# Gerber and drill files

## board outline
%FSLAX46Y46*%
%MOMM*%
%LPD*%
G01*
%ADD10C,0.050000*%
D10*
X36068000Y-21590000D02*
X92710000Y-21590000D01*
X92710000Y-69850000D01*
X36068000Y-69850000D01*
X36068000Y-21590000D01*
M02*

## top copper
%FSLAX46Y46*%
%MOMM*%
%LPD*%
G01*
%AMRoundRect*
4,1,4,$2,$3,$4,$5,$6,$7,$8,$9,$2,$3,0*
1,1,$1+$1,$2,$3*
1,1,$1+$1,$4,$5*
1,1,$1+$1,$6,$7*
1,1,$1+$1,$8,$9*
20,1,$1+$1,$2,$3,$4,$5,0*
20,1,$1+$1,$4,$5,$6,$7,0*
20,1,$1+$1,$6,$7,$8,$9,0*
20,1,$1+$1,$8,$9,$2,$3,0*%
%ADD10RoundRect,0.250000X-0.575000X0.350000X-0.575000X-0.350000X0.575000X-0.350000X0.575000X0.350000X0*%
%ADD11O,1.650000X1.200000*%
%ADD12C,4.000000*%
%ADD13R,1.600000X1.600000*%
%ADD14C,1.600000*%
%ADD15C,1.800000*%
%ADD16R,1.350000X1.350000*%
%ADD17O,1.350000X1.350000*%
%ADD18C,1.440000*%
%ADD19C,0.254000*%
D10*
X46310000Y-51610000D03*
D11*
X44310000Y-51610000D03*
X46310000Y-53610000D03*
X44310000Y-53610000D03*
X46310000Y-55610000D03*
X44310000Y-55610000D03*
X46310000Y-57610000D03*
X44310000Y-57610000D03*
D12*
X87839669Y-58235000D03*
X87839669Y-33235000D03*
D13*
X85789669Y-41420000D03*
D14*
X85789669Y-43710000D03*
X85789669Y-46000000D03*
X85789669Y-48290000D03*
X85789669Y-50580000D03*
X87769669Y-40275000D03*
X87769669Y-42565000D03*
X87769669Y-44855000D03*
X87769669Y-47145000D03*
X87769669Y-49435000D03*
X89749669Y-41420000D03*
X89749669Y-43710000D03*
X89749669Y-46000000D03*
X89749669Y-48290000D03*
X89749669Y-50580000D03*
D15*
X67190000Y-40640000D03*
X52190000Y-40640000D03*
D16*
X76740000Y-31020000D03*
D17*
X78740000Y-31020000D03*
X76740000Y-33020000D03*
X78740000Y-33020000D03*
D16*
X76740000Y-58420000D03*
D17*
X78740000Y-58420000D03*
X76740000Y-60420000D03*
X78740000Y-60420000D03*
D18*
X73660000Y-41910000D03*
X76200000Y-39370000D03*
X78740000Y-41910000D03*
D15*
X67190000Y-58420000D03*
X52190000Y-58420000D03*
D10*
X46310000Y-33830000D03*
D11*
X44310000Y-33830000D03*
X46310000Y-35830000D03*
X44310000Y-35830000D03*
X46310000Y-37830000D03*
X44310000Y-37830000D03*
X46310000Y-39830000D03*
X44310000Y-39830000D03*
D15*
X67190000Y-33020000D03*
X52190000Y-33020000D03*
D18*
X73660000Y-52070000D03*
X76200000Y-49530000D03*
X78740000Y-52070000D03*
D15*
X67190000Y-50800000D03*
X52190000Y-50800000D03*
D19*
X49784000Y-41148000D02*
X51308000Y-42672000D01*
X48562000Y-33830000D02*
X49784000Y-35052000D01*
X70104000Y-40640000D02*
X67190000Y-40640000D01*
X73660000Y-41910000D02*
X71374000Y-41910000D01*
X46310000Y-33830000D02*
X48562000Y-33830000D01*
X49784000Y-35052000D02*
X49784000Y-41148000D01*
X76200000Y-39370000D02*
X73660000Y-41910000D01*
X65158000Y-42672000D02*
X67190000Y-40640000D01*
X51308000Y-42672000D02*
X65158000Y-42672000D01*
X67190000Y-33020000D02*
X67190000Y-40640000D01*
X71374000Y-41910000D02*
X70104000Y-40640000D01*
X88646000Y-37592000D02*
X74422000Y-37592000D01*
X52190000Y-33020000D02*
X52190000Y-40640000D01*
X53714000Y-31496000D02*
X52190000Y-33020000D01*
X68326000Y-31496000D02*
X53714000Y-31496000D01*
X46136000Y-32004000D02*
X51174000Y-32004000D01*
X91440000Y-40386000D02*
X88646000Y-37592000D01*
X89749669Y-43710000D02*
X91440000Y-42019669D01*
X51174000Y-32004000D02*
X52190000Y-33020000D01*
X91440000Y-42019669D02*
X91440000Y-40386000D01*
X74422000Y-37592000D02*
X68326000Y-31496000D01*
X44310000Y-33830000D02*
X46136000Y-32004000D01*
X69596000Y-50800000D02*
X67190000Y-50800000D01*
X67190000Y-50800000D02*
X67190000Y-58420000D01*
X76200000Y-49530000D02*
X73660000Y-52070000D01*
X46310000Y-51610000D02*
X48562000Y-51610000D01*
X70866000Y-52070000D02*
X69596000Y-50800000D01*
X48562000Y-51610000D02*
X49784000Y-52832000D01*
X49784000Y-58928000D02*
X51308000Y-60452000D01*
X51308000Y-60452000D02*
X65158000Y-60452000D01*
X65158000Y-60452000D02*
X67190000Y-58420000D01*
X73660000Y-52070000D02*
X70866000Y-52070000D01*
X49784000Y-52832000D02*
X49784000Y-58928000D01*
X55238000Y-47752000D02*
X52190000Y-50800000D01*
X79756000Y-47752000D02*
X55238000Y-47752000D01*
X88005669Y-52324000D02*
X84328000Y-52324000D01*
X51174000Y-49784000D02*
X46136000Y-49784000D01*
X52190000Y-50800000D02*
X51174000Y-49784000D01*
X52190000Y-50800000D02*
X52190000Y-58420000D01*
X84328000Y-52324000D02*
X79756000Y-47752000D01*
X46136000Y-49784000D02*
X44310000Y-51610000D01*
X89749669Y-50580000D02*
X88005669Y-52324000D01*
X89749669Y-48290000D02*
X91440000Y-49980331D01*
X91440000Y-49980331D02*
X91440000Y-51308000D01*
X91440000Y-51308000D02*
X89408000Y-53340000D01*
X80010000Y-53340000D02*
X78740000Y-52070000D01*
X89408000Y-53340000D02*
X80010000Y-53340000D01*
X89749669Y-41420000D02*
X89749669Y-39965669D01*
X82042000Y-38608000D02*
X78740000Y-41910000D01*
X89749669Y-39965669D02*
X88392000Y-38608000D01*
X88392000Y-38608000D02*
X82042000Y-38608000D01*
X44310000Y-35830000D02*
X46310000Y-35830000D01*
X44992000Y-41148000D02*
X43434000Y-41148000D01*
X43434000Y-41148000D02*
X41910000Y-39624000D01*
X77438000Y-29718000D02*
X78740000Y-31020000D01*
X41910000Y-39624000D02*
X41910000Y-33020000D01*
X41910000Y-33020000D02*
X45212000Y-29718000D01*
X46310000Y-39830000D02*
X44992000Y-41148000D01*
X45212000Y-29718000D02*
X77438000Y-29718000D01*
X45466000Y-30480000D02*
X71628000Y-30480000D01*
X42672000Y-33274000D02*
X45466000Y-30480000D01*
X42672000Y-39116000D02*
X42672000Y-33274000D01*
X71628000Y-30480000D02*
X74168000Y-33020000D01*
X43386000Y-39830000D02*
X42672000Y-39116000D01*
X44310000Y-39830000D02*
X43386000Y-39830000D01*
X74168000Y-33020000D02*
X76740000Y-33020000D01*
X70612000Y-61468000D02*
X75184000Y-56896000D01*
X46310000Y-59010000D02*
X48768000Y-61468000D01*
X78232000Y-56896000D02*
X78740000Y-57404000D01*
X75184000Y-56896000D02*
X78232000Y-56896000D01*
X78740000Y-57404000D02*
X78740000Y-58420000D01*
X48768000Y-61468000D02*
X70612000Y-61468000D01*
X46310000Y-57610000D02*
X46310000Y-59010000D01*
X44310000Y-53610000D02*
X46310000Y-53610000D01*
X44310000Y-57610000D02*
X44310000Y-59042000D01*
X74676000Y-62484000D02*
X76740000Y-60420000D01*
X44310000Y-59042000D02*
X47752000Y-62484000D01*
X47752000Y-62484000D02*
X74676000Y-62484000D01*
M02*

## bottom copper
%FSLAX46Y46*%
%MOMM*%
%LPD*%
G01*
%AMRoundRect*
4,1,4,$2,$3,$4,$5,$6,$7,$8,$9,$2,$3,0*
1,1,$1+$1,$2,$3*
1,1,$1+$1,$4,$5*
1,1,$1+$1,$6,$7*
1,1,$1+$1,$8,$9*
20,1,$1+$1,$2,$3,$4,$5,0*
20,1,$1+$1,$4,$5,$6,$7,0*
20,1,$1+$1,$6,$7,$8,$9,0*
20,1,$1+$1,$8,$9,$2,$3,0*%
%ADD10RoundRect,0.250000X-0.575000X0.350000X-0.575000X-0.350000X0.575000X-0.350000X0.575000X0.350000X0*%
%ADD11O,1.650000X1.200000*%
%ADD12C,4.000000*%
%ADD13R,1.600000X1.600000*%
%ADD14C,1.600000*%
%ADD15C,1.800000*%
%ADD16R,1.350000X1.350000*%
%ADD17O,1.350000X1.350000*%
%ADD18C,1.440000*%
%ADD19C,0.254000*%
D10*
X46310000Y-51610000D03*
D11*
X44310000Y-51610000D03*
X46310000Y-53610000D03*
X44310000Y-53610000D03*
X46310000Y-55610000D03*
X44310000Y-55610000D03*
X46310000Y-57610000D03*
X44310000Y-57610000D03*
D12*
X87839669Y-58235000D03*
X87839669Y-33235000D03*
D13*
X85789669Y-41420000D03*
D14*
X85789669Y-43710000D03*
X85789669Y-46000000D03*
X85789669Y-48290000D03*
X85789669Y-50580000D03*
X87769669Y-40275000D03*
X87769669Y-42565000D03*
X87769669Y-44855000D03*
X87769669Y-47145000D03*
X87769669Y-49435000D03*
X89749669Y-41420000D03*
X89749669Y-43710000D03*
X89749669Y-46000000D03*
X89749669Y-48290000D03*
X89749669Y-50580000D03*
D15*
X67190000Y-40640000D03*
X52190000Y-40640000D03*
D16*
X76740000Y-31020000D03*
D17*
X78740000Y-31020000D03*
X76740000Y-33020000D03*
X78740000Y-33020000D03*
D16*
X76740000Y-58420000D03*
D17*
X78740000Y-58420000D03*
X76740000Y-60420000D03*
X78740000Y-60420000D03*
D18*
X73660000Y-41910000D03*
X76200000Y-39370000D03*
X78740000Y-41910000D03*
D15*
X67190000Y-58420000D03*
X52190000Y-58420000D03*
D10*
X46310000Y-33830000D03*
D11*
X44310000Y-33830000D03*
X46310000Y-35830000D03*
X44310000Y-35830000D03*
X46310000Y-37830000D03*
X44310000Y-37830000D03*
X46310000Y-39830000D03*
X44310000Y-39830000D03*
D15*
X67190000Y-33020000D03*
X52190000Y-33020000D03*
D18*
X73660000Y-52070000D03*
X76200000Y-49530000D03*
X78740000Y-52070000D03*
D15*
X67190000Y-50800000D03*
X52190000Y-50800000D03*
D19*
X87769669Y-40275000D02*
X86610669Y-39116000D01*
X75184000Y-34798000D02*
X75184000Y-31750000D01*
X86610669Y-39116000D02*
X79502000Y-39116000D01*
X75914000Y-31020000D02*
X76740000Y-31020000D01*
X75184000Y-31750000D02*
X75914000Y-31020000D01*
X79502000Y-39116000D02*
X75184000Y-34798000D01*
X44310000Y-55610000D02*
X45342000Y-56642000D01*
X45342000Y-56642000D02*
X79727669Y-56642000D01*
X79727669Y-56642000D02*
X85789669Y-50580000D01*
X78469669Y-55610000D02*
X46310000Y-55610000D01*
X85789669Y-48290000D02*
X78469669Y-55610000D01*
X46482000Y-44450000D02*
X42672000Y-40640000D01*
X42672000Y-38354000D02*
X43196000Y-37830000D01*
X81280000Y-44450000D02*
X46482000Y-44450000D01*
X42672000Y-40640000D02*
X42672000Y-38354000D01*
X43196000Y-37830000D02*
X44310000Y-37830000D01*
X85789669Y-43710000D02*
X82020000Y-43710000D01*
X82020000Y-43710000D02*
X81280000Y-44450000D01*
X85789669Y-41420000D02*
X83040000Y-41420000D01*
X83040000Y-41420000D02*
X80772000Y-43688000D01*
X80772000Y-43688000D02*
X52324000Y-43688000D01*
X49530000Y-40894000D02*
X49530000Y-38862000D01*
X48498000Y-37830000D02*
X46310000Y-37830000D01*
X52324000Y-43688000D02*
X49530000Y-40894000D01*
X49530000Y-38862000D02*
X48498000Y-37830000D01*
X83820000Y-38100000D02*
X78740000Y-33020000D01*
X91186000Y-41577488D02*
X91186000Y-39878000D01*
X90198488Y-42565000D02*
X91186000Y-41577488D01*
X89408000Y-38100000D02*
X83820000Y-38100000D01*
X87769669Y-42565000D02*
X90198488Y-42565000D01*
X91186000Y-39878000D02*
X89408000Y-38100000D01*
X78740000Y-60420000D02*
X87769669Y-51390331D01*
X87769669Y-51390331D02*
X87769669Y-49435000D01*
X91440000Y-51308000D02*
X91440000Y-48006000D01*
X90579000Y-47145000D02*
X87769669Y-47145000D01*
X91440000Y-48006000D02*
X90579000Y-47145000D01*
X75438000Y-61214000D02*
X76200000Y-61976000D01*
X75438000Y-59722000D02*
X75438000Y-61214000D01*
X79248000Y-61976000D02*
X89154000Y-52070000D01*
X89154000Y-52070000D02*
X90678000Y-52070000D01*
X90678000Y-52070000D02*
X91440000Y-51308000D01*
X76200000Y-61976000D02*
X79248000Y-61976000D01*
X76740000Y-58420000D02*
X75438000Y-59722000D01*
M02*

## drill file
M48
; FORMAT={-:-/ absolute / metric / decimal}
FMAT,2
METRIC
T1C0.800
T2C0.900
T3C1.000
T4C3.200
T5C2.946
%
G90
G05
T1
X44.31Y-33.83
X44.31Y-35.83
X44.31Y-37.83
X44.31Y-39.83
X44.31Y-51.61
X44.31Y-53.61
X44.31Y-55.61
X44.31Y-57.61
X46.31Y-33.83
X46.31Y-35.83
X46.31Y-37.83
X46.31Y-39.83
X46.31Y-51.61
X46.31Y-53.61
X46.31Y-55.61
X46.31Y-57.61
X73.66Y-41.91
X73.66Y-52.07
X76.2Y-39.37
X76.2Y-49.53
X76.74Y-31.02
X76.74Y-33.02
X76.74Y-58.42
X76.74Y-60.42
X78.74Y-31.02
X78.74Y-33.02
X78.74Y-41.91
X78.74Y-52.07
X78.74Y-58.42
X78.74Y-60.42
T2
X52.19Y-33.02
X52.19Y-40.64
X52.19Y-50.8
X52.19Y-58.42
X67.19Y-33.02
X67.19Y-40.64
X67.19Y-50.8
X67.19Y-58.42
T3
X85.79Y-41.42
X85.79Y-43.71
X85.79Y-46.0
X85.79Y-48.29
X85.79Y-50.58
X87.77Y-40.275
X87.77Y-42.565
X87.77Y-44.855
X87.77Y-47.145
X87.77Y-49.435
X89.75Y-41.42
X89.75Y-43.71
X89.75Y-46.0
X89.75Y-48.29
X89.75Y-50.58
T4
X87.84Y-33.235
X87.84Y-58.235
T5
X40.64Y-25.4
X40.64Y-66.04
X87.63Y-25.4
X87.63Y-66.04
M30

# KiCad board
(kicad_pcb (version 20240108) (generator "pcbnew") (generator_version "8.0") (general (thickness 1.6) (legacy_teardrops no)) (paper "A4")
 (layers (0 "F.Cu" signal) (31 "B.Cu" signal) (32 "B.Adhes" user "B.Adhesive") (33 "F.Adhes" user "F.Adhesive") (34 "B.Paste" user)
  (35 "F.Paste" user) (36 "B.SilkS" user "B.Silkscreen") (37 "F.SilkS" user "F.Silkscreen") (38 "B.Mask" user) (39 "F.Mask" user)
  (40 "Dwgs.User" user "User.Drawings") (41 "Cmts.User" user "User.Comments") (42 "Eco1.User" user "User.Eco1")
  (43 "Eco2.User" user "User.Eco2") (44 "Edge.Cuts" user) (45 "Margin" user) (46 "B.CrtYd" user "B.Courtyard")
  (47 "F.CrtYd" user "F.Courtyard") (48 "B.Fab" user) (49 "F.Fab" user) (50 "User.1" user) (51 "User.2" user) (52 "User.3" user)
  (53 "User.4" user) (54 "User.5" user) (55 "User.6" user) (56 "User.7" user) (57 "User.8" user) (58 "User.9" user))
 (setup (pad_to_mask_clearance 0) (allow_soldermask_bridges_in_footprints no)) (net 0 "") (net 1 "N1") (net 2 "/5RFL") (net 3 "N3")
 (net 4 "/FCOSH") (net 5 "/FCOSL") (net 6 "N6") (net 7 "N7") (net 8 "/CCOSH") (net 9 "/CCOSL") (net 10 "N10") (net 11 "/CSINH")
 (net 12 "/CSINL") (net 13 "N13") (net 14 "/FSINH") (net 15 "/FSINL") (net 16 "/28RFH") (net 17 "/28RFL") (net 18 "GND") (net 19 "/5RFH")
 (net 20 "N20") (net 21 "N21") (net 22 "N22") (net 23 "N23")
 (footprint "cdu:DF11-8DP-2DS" (layer "F.Cu") (at 46.31 51.61 90)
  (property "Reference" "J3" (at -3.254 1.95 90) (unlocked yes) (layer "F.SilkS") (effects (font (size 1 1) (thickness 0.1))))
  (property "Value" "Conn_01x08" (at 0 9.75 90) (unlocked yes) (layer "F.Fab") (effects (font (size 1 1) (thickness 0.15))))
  (pad "1" thru_hole roundrect (at 0 0 270) (size 1.2 1.65) (drill 0.8) (layers "*.Cu" "*.Mask") (remove_unused_layers no)
   (roundrect_rratio 0.2083333333) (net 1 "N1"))
  (pad "2" thru_hole oval (at 0 -2 270) (size 1.2 1.65) (drill 0.8) (layers "*.Cu" "*.Mask") (remove_unused_layers no) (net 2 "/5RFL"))
  (pad "3" thru_hole oval (at -2 0 270) (size 1.2 1.65) (drill 0.8) (layers "*.Cu" "*.Mask") (remove_unused_layers no) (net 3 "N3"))
  (pad "4" thru_hole oval (at -2 -2 270) (size 1.2 1.65) (drill 0.8) (layers "*.Cu" "*.Mask") (remove_unused_layers no) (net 3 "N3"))
  (pad "5" thru_hole oval (at -4 0 270) (size 1.2 1.65) (drill 0.8) (layers "*.Cu" "*.Mask") (remove_unused_layers no) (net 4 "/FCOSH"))
  (pad "6" thru_hole oval (at -4 -2 270) (size 1.2 1.65) (drill 0.8) (layers "*.Cu" "*.Mask") (remove_unused_layers no) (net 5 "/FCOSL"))
  (pad "7" thru_hole oval (at -6 0 270) (size 1.2 1.65) (drill 0.8) (layers "*.Cu" "*.Mask") (remove_unused_layers no) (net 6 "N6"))
  (pad "8" thru_hole oval (at -6 -2 270) (size 1.2 1.65) (drill 0.8) (layers "*.Cu" "*.Mask") (remove_unused_layers no) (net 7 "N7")))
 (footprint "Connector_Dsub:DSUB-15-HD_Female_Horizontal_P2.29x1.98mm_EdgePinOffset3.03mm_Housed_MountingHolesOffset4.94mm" (layer "F.Cu")
  (at 85.789669 41.42 90)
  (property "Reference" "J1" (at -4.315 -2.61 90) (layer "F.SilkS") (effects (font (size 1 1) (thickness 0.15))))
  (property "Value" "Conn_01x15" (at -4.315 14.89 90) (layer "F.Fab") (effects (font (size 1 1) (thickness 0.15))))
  (pad "0" thru_hole circle (at -16.815 2.05 90) (size 4 4) (drill 3.2) (layers "*.Cu" "*.Mask") (remove_unused_layers no))
  (pad "0" thru_hole circle (at 8.185 2.05 90) (size 4 4) (drill 3.2) (layers "*.Cu" "*.Mask") (remove_unused_layers no))
  (pad "1" thru_hole rect (at 0 0 90) (size 1.6 1.6) (drill 1) (layers "*.Cu" "*.Mask") (remove_unused_layers no) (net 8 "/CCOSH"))
  (pad "2" thru_hole circle (at -2.29 0 90) (size 1.6 1.6) (drill 1) (layers "*.Cu" "*.Mask") (remove_unused_layers no) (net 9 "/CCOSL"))
  (pad "3" thru_hole circle (at -4.58 0 90) (size 1.6 1.6) (drill 1) (layers "*.Cu" "*.Mask") (remove_unused_layers no) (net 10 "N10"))
  (pad "4" thru_hole circle (at -6.87 0 90) (size 1.6 1.6) (drill 1) (layers "*.Cu" "*.Mask") (remove_unused_layers no) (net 4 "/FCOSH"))
  (pad "5" thru_hole circle (at -9.16 0 90) (size 1.6 1.6) (drill 1) (layers "*.Cu" "*.Mask") (remove_unused_layers no) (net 5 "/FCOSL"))
  (pad "6" thru_hole circle (at 1.145 1.98 90) (size 1.6 1.6) (drill 1) (layers "*.Cu" "*.Mask") (remove_unused_layers no) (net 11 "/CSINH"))
  (pad "7" thru_hole circle (at -1.145 1.98 90) (size 1.6 1.6) (drill 1) (layers "*.Cu" "*.Mask") (remove_unused_layers no)
   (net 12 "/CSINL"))
  (pad "8" thru_hole circle (at -3.435 1.98 90) (size 1.6 1.6) (drill 1) (layers "*.Cu" "*.Mask") (remove_unused_layers no) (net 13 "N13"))
  (pad "9" thru_hole circle (at -5.725 1.98 90) (size 1.6 1.6) (drill 1) (layers "*.Cu" "*.Mask") (remove_unused_layers no)
   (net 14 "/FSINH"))
  (pad "10" thru_hole circle (at -8.015 1.98 90) (size 1.6 1.6) (drill 1) (layers "*.Cu" "*.Mask") (remove_unused_layers no)
   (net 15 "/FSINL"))
  (pad "11" thru_hole circle (at 0 3.96 90) (size 1.6 1.6) (drill 1) (layers "*.Cu" "*.Mask") (remove_unused_layers no) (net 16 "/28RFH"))
  (pad "12" thru_hole circle (at -2.29 3.96 90) (size 1.6 1.6) (drill 1) (layers "*.Cu" "*.Mask") (remove_unused_layers no)
   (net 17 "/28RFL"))
  (pad "13" thru_hole circle (at -4.58 3.96 90) (size 1.6 1.6) (drill 1) (layers "*.Cu" "*.Mask") (remove_unused_layers no) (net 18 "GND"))
  (pad "14" thru_hole circle (at -6.87 3.96 90) (size 1.6 1.6) (drill 1) (layers "*.Cu" "*.Mask") (remove_unused_layers no) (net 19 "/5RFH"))
  (pad "15" thru_hole circle (at -9.16 3.96 90) (size 1.6 1.6) (drill 1) (layers "*.Cu" "*.Mask") (remove_unused_layers no) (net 2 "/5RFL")))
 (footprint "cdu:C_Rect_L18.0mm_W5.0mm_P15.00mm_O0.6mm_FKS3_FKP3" (layer "F.Cu") (at 67.19 40.64 180)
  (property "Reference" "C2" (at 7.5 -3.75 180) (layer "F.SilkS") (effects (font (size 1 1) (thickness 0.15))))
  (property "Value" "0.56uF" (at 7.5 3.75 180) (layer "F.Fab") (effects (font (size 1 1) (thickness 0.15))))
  (pad "1" thru_hole circle (at 0 0 180) (size 1.8 1.8) (drill 0.9) (layers "*.Cu" "*.Mask") (remove_unused_layers no) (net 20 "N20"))
  (pad "2" thru_hole circle (at 15 0 180) (size 1.8 1.8) (drill 0.9) (layers "*.Cu" "*.Mask") (remove_unused_layers no) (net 17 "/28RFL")))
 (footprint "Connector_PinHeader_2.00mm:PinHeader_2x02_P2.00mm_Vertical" (layer "F.Cu") (at 76.74 31.02)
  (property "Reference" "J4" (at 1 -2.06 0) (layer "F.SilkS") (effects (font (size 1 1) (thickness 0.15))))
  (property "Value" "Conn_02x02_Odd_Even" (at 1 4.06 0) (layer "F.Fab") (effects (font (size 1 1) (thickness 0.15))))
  (pad "1" thru_hole rect (at 0 0) (size 1.35 1.35) (drill 0.8) (layers "*.Cu" "*.Mask") (remove_unused_layers no) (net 11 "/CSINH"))
  (pad "2" thru_hole oval (at 2 0) (size 1.35 1.35) (drill 0.8) (layers "*.Cu" "*.Mask") (remove_unused_layers no) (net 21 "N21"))
  (pad "3" thru_hole oval (at 0 2) (size 1.35 1.35) (drill 0.8) (layers "*.Cu" "*.Mask") (remove_unused_layers no) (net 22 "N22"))
  (pad "4" thru_hole oval (at 2 2) (size 1.35 1.35) (drill 0.8) (layers "*.Cu" "*.Mask") (remove_unused_layers no) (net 12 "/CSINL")))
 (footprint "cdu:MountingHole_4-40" (layer "F.Cu") (at 87.63 25.4)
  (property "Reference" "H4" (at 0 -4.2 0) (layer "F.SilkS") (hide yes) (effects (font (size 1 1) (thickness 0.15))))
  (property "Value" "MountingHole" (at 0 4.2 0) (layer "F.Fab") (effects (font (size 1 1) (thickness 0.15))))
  (pad "" np_thru_hole circle (at 0 0) (size 2.9464 2.9464) (drill 2.9464) (layers "F&B.Cu" "*.Mask")))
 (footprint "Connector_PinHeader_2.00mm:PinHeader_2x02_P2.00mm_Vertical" (layer "F.Cu") (at 76.74 58.42)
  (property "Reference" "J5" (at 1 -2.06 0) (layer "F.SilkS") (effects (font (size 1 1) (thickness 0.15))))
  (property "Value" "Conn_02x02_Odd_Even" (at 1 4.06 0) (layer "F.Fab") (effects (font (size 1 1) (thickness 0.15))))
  (pad "1" thru_hole rect (at 0 0) (size 1.35 1.35) (drill 0.8) (layers "*.Cu" "*.Mask") (remove_unused_layers no) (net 14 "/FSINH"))
  (pad "2" thru_hole oval (at 2 0) (size 1.35 1.35) (drill 0.8) (layers "*.Cu" "*.Mask") (remove_unused_layers no) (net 6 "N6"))
  (pad "3" thru_hole oval (at 0 2) (size 1.35 1.35) (drill 0.8) (layers "*.Cu" "*.Mask") (remove_unused_layers no) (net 7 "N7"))
  (pad "4" thru_hole oval (at 2 2) (size 1.35 1.35) (drill 0.8) (layers "*.Cu" "*.Mask") (remove_unused_layers no) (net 15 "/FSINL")))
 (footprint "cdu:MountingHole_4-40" (layer "F.Cu") (at 40.64 25.4)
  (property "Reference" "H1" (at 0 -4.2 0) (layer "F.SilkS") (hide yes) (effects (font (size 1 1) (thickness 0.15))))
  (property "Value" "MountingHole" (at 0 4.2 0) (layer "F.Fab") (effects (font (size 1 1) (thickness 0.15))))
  (pad "" np_thru_hole circle (at 0 0) (size 2.9464 2.9464) (drill 2.9464) (layers "F&B.Cu" "*.Mask")))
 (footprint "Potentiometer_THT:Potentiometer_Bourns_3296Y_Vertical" (layer "F.Cu") (at 73.66 41.91 180)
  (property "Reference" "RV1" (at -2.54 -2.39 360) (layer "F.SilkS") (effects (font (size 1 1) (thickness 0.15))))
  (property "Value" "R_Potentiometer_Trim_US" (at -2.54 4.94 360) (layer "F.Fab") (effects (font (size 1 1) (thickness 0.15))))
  (pad "1" thru_hole circle (at 0 0 180) (size 1.44 1.44) (drill 0.8) (layers "*.Cu" "*.Mask") (remove_unused_layers no) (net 20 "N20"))
  (pad "2" thru_hole circle (at -2.54 2.54 180) (size 1.44 1.44) (drill 0.8) (layers "*.Cu" "*.Mask") (remove_unused_layers no)
   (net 20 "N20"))
  (pad "3" thru_hole circle (at -5.08 0 180) (size 1.44 1.44) (drill 0.8) (layers "*.Cu" "*.Mask") (remove_unused_layers no)
   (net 16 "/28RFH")))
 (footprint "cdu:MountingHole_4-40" (layer "F.Cu") (at 40.64 66.04)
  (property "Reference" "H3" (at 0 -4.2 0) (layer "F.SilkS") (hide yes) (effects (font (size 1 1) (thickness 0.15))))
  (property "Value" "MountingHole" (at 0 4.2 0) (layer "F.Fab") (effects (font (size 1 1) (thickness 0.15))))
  (pad "" np_thru_hole circle (at 0 0) (size 2.9464 2.9464) (drill 2.9464) (layers "F&B.Cu" "*.Mask")))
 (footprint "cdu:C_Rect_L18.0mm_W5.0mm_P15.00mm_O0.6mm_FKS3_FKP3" (layer "F.Cu") (at 67.19 58.42 180)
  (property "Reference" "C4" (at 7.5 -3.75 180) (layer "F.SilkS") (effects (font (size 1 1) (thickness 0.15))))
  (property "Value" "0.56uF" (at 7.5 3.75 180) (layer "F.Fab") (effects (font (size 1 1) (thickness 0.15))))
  (pad "1" thru_hole circle (at 0 0 180) (size 1.8 1.8) (drill 0.9) (layers "*.Cu" "*.Mask") (remove_unused_layers no) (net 1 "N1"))
  (pad "2" thru_hole circle (at 15 0 180) (size 1.8 1.8) (drill 0.9) (layers "*.Cu" "*.Mask") (remove_unused_layers no) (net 2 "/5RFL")))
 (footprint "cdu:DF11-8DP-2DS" (layer "F.Cu") (at 46.31 33.83 90)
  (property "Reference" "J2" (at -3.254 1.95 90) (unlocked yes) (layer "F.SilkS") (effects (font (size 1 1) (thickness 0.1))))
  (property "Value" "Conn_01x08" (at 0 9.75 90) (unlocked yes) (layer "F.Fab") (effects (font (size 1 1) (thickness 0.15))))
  (pad "1" thru_hole roundrect (at 0 0 270) (size 1.2 1.65) (drill 0.8) (layers "*.Cu" "*.Mask") (remove_unused_layers no)
   (roundrect_rratio 0.2083333333) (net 20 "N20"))
  (pad "2" thru_hole oval (at 0 -2 270) (size 1.2 1.65) (drill 0.8) (layers "*.Cu" "*.Mask") (remove_unused_layers no) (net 17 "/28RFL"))
  (pad "3" thru_hole oval (at -2 0 270) (size 1.2 1.65) (drill 0.8) (layers "*.Cu" "*.Mask") (remove_unused_layers no) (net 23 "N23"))
  (pad "4" thru_hole oval (at -2 -2 270) (size 1.2 1.65) (drill 0.8) (layers "*.Cu" "*.Mask") (remove_unused_layers no) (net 23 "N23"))
  (pad "5" thru_hole oval (at -4 0 270) (size 1.2 1.65) (drill 0.8) (layers "*.Cu" "*.Mask") (remove_unused_layers no) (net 8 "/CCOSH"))
  (pad "6" thru_hole oval (at -4 -2 270) (size 1.2 1.65) (drill 0.8) (layers "*.Cu" "*.Mask") (remove_unused_layers no) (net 9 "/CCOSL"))
  (pad "7" thru_hole oval (at -6 0 270) (size 1.2 1.65) (drill 0.8) (layers "*.Cu" "*.Mask") (remove_unused_layers no) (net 21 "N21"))
  (pad "8" thru_hole oval (at -6 -2 270) (size 1.2 1.65) (drill 0.8) (layers "*.Cu" "*.Mask") (remove_unused_layers no) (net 22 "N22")))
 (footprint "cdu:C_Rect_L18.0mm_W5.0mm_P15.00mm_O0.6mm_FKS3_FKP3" (layer "F.Cu") (at 67.19 33.02 180)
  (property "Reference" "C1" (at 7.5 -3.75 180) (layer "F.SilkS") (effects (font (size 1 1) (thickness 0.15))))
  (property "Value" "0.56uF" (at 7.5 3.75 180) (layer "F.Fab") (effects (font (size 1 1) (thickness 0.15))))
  (pad "1" thru_hole circle (at 0 0 180) (size 1.8 1.8) (drill 0.9) (layers "*.Cu" "*.Mask") (remove_unused_layers no) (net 20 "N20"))
  (pad "2" thru_hole circle (at 15 0 180) (size 1.8 1.8) (drill 0.9) (layers "*.Cu" "*.Mask") (remove_unused_layers no) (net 17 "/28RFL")))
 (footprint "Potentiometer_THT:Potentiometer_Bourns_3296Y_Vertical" (layer "F.Cu") (at 73.66 52.07 180)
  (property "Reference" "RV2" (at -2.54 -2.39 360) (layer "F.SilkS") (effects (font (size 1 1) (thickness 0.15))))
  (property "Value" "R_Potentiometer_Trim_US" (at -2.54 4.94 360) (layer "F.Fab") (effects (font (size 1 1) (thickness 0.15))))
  (pad "1" thru_hole circle (at 0 0 180) (size 1.44 1.44) (drill 0.8) (layers "*.Cu" "*.Mask") (remove_unused_layers no) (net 1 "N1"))
  (pad "2" thru_hole circle (at -2.54 2.54 180) (size 1.44 1.44) (drill 0.8) (layers "*.Cu" "*.Mask") (remove_unused_layers no) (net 1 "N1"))
  (pad "3" thru_hole circle (at -5.08 0 180) (size 1.44 1.44) (drill 0.8) (layers "*.Cu" "*.Mask") (remove_unused_layers no)
   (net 19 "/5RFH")))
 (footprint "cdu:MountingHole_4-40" (layer "F.Cu") (at 87.63 66.04)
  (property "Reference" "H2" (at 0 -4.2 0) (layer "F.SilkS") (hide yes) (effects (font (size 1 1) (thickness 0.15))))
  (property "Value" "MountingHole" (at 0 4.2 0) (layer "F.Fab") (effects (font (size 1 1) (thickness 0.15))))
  (pad "" np_thru_hole circle (at 0 0) (size 2.9464 2.9464) (drill 2.9464) (layers "F&B.Cu" "*.Mask")))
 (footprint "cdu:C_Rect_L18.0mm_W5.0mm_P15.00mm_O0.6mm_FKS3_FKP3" (layer "F.Cu") (at 67.19 50.8 180)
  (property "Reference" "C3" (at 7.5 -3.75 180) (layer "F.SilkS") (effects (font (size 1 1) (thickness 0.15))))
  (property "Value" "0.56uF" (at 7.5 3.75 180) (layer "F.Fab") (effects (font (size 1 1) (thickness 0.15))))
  (pad "1" thru_hole circle (at 0 0 180) (size 1.8 1.8) (drill 0.9) (layers "*.Cu" "*.Mask") (remove_unused_layers no) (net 1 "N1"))
  (pad "2" thru_hole circle (at 15 0 180) (size 1.8 1.8) (drill 0.9) (layers "*.Cu" "*.Mask") (remove_unused_layers no) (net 2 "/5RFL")))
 (gr_rect (start 36.068 21.59) (end 92.71 69.85) (stroke (width 0.05) (type default)) (fill none) (layer "Edge.Cuts"))
 (segment (start 49.784 41.148) (end 51.308 42.672) (width 0.254) (layer "F.Cu") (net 20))
 (segment (start 48.562 33.83) (end 49.784 35.052) (width 0.254) (layer "F.Cu") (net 20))
 (segment (start 70.104 40.64) (end 67.19 40.64) (width 0.254) (layer "F.Cu") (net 20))
 (segment (start 73.66 41.91) (end 71.374 41.91) (width 0.254) (layer "F.Cu") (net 20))
 (segment (start 46.31 33.83) (end 48.562 33.83) (width 0.254) (layer "F.Cu") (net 20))
 (segment (start 49.784 35.052) (end 49.784 41.148) (width 0.254) (layer "F.Cu") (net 20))
 (segment (start 76.2 39.37) (end 73.66 41.91) (width 0.254) (layer "F.Cu") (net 20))
 (segment (start 65.158 42.672) (end 67.19 40.64) (width 0.254) (layer "F.Cu") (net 20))
 (segment (start 51.308 42.672) (end 65.158 42.672) (width 0.254) (layer "F.Cu") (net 20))
 (segment (start 67.19 33.02) (end 67.19 40.64) (width 0.254) (layer "F.Cu") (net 20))
 (segment (start 71.374 41.91) (end 70.104 40.64) (width 0.254) (layer "F.Cu") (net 20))
 (segment (start 88.646 37.592) (end 74.422 37.592) (width 0.254) (layer "F.Cu") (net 17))
 (segment (start 52.19 33.02) (end 52.19 40.64) (width 0.254) (layer "F.Cu") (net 17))
 (segment (start 53.714 31.496) (end 52.19 33.02) (width 0.254) (layer "F.Cu") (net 17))
 (segment (start 68.326 31.496) (end 53.714 31.496) (width 0.254) (layer "F.Cu") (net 17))
 (segment (start 46.136 32.004) (end 51.174 32.004) (width 0.254) (layer "F.Cu") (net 17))
 (segment (start 91.44 40.386) (end 88.646 37.592) (width 0.254) (layer "F.Cu") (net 17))
 (segment (start 89.749669 43.71) (end 91.44 42.019669) (width 0.254) (layer "F.Cu") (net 17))
 (segment (start 51.174 32.004) (end 52.19 33.02) (width 0.254) (layer "F.Cu") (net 17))
 (segment (start 91.44 42.019669) (end 91.44 40.386) (width 0.254) (layer "F.Cu") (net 17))
 (segment (start 74.422 37.592) (end 68.326 31.496) (width 0.254) (layer "F.Cu") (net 17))
 (segment (start 44.31 33.83) (end 46.136 32.004) (width 0.254) (layer "F.Cu") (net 17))
 (segment (start 69.596 50.8) (end 67.19 50.8) (width 0.254) (layer "F.Cu") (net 1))
 (segment (start 67.19 50.8) (end 67.19 58.42) (width 0.254) (layer "F.Cu") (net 1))
 (segment (start 76.2 49.53) (end 73.66 52.07) (width 0.254) (layer "F.Cu") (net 1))
 (segment (start 46.31 51.61) (end 48.562 51.61) (width 0.254) (layer "F.Cu") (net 1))
 (segment (start 70.866 52.07) (end 69.596 50.8) (width 0.254) (layer "F.Cu") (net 1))
 (segment (start 48.562 51.61) (end 49.784 52.832) (width 0.254) (layer "F.Cu") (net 1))
 (segment (start 49.784 58.928) (end 51.308 60.452) (width 0.254) (layer "F.Cu") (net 1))
 (segment (start 51.308 60.452) (end 65.158 60.452) (width 0.254) (layer "F.Cu") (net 1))
 (segment (start 65.158 60.452) (end 67.19 58.42) (width 0.254) (layer "F.Cu") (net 1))
 (segment (start 73.66 52.07) (end 70.866 52.07) (width 0.254) (layer "F.Cu") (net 1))
 (segment (start 49.784 52.832) (end 49.784 58.928) (width 0.254) (layer "F.Cu") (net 1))
 (segment (start 55.238 47.752) (end 52.19 50.8) (width 0.254) (layer "F.Cu") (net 2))
 (segment (start 79.756 47.752) (end 55.238 47.752) (width 0.254) (layer "F.Cu") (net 2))
 (segment (start 88.005669 52.324) (end 84.328 52.324) (width 0.254) (layer "F.Cu") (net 2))
 (segment (start 51.174 49.784) (end 46.136 49.784) (width 0.254) (layer "F.Cu") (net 2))
 (segment (start 52.19 50.8) (end 51.174 49.784) (width 0.254) (layer "F.Cu") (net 2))
 (segment (start 52.19 50.8) (end 52.19 58.42) (width 0.254) (layer "F.Cu") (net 2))
 (segment (start 84.328 52.324) (end 79.756 47.752) (width 0.254) (layer "F.Cu") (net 2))
 (segment (start 46.136 49.784) (end 44.31 51.61) (width 0.254) (layer "F.Cu") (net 2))
 (segment (start 89.749669 50.58) (end 88.005669 52.324) (width 0.254) (layer "F.Cu") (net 2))
 (segment (start 87.769669 40.275) (end 86.610669 39.116) (width 0.254) (layer "B.Cu") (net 11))
 (segment (start 75.184 34.798) (end 75.184 31.75) (width 0.254) (layer "B.Cu") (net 11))
 (segment (start 86.610669 39.116) (end 79.502 39.116) (width 0.254) (layer "B.Cu") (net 11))
 (segment (start 75.914 31.02) (end 76.74 31.02) (width 0.254) (layer "B.Cu") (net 11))
 (segment (start 75.184 31.75) (end 75.914 31.02) (width 0.254) (layer "B.Cu") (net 11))
 (segment (start 79.502 39.116) (end 75.184 34.798) (width 0.254) (layer "B.Cu") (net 11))
 (segment (start 44.31 55.61) (end 45.342 56.642) (width 0.254) (layer "B.Cu") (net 5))
 (segment (start 45.342 56.642) (end 79.727669 56.642) (width 0.254) (layer "B.Cu") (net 5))
 (segment (start 79.727669 56.642) (end 85.789669 50.58) (width 0.254) (layer "B.Cu") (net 5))
 (segment (start 78.469669 55.61) (end 46.31 55.61) (width 0.254) (layer "B.Cu") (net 4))
 (segment (start 85.789669 48.29) (end 78.469669 55.61) (width 0.254) (layer "B.Cu") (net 4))
 (segment (start 46.482 44.45) (end 42.672 40.64) (width 0.254) (layer "B.Cu") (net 9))
 (segment (start 42.672 38.354) (end 43.196 37.83) (width 0.254) (layer "B.Cu") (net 9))
 (segment (start 81.28 44.45) (end 46.482 44.45) (width 0.254) (layer "B.Cu") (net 9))
 (segment (start 42.672 40.64) (end 42.672 38.354) (width 0.254) (layer "B.Cu") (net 9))
 (segment (start 43.196 37.83) (end 44.31 37.83) (width 0.254) (layer "B.Cu") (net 9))
 (segment (start 85.789669 43.71) (end 82.02 43.71) (width 0.254) (layer "B.Cu") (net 9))
 (segment (start 82.02 43.71) (end 81.28 44.45) (width 0.254) (layer "B.Cu") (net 9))
 (segment (start 85.789669 41.42) (end 83.04 41.42) (width 0.254) (layer "B.Cu") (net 8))
 (segment (start 83.04 41.42) (end 80.772 43.688) (width 0.254) (layer "B.Cu") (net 8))
 (segment (start 80.772 43.688) (end 52.324 43.688) (width 0.254) (layer "B.Cu") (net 8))
 (segment (start 49.53 40.894) (end 49.53 38.862) (width 0.254) (layer "B.Cu") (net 8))
 (segment (start 48.498 37.83) (end 46.31 37.83) (width 0.254) (layer "B.Cu") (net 8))
 (segment (start 52.324 43.688) (end 49.53 40.894) (width 0.254) (layer "B.Cu") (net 8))
 (segment (start 49.53 38.862) (end 48.498 37.83) (width 0.254) (layer "B.Cu") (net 8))
 (segment (start 83.82 38.1) (end 78.74 33.02) (width 0.254) (layer "B.Cu") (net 12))
 (segment (start 91.186 41.577488) (end 91.186 39.878) (width 0.254) (layer "B.Cu") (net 12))
 (segment (start 90.198488 42.565) (end 91.186 41.577488) (width 0.254) (layer "B.Cu") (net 12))
 (segment (start 89.408 38.1) (end 83.82 38.1) (width 0.254) (layer "B.Cu") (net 12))
 (segment (start 87.769669 42.565) (end 90.198488 42.565) (width 0.254) (layer "B.Cu") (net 12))
 (segment (start 91.186 39.878) (end 89.408 38.1) (width 0.254) (layer "B.Cu") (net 12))
 (segment (start 78.74 60.42) (end 87.769669 51.390331) (width 0.254) (layer "B.Cu") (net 15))
 (segment (start 87.769669 51.390331) (end 87.769669 49.435) (width 0.254) (layer "B.Cu") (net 15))
 (segment (start 89.749669 48.29) (end 91.44 49.980331) (width 0.254) (layer "F.Cu") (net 19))
 (segment (start 91.44 49.980331) (end 91.44 51.308) (width 0.254) (layer "F.Cu") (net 19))
 (segment (start 91.44 51.308) (end 89.408 53.34) (width 0.254) (layer "F.Cu") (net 19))
 (segment (start 80.01 53.34) (end 78.74 52.07) (width 0.254) (layer "F.Cu") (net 19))
 (segment (start 89.408 53.34) (end 80.01 53.34) (width 0.254) (layer "F.Cu") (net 19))
 (segment (start 91.44 51.308) (end 91.44 48.006) (width 0.254) (layer "B.Cu") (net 14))
 (segment (start 90.579 47.145) (end 87.769669 47.145) (width 0.254) (layer "B.Cu") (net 14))
 (segment (start 91.44 48.006) (end 90.579 47.145) (width 0.254) (layer "B.Cu") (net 14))
 (segment (start 75.438 61.214) (end 76.2 61.976) (width 0.254) (layer "B.Cu") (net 14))
 (segment (start 75.438 59.722) (end 75.438 61.214) (width 0.254) (layer "B.Cu") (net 14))
 (segment (start 79.248 61.976) (end 89.154 52.07) (width 0.254) (layer "B.Cu") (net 14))
 (segment (start 89.154 52.07) (end 90.678 52.07) (width 0.254) (layer "B.Cu") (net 14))
 (segment (start 90.678 52.07) (end 91.44 51.308) (width 0.254) (layer "B.Cu") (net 14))
 (segment (start 76.2 61.976) (end 79.248 61.976) (width 0.254) (layer "B.Cu") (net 14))
 (segment (start 76.74 58.42) (end 75.438 59.722) (width 0.254) (layer "B.Cu") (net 14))
 (segment (start 89.749669 41.42) (end 89.749669 39.965669) (width 0.254) (layer "F.Cu") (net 16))
 (segment (start 82.042 38.608) (end 78.74 41.91) (width 0.254) (layer "F.Cu") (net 16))
 (segment (start 89.749669 39.965669) (end 88.392 38.608) (width 0.254) (layer "F.Cu") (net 16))
 (segment (start 88.392 38.608) (end 82.042 38.608) (width 0.254) (layer "F.Cu") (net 16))
 (segment (start 44.31 35.83) (end 46.31 35.83) (width 0.254) (layer "F.Cu") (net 23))
 (segment (start 44.992 41.148) (end 43.434 41.148) (width 0.254) (layer "F.Cu") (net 21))
 (segment (start 43.434 41.148) (end 41.91 39.624) (width 0.254) (layer "F.Cu") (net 21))
 (segment (start 77.438 29.718) (end 78.74 31.02) (width 0.254) (layer "F.Cu") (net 21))
 (segment (start 41.91 39.624) (end 41.91 33.02) (width 0.254) (layer "F.Cu") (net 21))
 (segment (start 41.91 33.02) (end 45.212 29.718) (width 0.254) (layer "F.Cu") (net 21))
 (segment (start 46.31 39.83) (end 44.992 41.148) (width 0.254) (layer "F.Cu") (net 21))
 (segment (start 45.212 29.718) (end 77.438 29.718) (width 0.254) (layer "F.Cu") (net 21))
 (segment (start 45.466 30.48) (end 71.628 30.48) (width 0.254) (layer "F.Cu") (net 22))
 (segment (start 42.672 33.274) (end 45.466 30.48) (width 0.254) (layer "F.Cu") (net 22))
 (segment (start 42.672 39.116) (end 42.672 33.274) (width 0.254) (layer "F.Cu") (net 22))
 (segment (start 71.628 30.48) (end 74.168 33.02) (width 0.254) (layer "F.Cu") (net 22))
 (segment (start 43.386 39.83) (end 42.672 39.116) (width 0.254) (layer "F.Cu") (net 22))
 (segment (start 44.31 39.83) (end 43.386 39.83) (width 0.254) (layer "F.Cu") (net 22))
 (segment (start 74.168 33.02) (end 76.74 33.02) (width 0.254) (layer "F.Cu") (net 22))
 (segment (start 70.612 61.468) (end 75.184 56.896) (width 0.254) (layer "F.Cu") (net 6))
 (segment (start 46.31 59.01) (end 48.768 61.468) (width 0.254) (layer "F.Cu") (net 6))
 (segment (start 78.232 56.896) (end 78.74 57.404) (width 0.254) (layer "F.Cu") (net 6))
 (segment (start 75.184 56.896) (end 78.232 56.896) (width 0.254) (layer "F.Cu") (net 6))
 (segment (start 78.74 57.404) (end 78.74 58.42) (width 0.254) (layer "F.Cu") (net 6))
 (segment (start 48.768 61.468) (end 70.612 61.468) (width 0.254) (layer "F.Cu") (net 6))
 (segment (start 46.31 57.61) (end 46.31 59.01) (width 0.254) (layer "F.Cu") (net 6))
 (segment (start 44.31 53.61) (end 46.31 53.61) (width 0.254) (layer "F.Cu") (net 3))
 (segment (start 44.31 57.61) (end 44.31 59.042) (width 0.254) (layer "F.Cu") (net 7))
 (segment (start 74.676 62.484) (end 76.74 60.42) (width 0.254) (layer "F.Cu") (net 7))
 (segment (start 44.31 59.042) (end 47.752 62.484) (width 0.254) (layer "F.Cu") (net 7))
 (segment (start 47.752 62.484) (end 74.676 62.484) (width 0.254) (layer "F.Cu") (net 7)))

